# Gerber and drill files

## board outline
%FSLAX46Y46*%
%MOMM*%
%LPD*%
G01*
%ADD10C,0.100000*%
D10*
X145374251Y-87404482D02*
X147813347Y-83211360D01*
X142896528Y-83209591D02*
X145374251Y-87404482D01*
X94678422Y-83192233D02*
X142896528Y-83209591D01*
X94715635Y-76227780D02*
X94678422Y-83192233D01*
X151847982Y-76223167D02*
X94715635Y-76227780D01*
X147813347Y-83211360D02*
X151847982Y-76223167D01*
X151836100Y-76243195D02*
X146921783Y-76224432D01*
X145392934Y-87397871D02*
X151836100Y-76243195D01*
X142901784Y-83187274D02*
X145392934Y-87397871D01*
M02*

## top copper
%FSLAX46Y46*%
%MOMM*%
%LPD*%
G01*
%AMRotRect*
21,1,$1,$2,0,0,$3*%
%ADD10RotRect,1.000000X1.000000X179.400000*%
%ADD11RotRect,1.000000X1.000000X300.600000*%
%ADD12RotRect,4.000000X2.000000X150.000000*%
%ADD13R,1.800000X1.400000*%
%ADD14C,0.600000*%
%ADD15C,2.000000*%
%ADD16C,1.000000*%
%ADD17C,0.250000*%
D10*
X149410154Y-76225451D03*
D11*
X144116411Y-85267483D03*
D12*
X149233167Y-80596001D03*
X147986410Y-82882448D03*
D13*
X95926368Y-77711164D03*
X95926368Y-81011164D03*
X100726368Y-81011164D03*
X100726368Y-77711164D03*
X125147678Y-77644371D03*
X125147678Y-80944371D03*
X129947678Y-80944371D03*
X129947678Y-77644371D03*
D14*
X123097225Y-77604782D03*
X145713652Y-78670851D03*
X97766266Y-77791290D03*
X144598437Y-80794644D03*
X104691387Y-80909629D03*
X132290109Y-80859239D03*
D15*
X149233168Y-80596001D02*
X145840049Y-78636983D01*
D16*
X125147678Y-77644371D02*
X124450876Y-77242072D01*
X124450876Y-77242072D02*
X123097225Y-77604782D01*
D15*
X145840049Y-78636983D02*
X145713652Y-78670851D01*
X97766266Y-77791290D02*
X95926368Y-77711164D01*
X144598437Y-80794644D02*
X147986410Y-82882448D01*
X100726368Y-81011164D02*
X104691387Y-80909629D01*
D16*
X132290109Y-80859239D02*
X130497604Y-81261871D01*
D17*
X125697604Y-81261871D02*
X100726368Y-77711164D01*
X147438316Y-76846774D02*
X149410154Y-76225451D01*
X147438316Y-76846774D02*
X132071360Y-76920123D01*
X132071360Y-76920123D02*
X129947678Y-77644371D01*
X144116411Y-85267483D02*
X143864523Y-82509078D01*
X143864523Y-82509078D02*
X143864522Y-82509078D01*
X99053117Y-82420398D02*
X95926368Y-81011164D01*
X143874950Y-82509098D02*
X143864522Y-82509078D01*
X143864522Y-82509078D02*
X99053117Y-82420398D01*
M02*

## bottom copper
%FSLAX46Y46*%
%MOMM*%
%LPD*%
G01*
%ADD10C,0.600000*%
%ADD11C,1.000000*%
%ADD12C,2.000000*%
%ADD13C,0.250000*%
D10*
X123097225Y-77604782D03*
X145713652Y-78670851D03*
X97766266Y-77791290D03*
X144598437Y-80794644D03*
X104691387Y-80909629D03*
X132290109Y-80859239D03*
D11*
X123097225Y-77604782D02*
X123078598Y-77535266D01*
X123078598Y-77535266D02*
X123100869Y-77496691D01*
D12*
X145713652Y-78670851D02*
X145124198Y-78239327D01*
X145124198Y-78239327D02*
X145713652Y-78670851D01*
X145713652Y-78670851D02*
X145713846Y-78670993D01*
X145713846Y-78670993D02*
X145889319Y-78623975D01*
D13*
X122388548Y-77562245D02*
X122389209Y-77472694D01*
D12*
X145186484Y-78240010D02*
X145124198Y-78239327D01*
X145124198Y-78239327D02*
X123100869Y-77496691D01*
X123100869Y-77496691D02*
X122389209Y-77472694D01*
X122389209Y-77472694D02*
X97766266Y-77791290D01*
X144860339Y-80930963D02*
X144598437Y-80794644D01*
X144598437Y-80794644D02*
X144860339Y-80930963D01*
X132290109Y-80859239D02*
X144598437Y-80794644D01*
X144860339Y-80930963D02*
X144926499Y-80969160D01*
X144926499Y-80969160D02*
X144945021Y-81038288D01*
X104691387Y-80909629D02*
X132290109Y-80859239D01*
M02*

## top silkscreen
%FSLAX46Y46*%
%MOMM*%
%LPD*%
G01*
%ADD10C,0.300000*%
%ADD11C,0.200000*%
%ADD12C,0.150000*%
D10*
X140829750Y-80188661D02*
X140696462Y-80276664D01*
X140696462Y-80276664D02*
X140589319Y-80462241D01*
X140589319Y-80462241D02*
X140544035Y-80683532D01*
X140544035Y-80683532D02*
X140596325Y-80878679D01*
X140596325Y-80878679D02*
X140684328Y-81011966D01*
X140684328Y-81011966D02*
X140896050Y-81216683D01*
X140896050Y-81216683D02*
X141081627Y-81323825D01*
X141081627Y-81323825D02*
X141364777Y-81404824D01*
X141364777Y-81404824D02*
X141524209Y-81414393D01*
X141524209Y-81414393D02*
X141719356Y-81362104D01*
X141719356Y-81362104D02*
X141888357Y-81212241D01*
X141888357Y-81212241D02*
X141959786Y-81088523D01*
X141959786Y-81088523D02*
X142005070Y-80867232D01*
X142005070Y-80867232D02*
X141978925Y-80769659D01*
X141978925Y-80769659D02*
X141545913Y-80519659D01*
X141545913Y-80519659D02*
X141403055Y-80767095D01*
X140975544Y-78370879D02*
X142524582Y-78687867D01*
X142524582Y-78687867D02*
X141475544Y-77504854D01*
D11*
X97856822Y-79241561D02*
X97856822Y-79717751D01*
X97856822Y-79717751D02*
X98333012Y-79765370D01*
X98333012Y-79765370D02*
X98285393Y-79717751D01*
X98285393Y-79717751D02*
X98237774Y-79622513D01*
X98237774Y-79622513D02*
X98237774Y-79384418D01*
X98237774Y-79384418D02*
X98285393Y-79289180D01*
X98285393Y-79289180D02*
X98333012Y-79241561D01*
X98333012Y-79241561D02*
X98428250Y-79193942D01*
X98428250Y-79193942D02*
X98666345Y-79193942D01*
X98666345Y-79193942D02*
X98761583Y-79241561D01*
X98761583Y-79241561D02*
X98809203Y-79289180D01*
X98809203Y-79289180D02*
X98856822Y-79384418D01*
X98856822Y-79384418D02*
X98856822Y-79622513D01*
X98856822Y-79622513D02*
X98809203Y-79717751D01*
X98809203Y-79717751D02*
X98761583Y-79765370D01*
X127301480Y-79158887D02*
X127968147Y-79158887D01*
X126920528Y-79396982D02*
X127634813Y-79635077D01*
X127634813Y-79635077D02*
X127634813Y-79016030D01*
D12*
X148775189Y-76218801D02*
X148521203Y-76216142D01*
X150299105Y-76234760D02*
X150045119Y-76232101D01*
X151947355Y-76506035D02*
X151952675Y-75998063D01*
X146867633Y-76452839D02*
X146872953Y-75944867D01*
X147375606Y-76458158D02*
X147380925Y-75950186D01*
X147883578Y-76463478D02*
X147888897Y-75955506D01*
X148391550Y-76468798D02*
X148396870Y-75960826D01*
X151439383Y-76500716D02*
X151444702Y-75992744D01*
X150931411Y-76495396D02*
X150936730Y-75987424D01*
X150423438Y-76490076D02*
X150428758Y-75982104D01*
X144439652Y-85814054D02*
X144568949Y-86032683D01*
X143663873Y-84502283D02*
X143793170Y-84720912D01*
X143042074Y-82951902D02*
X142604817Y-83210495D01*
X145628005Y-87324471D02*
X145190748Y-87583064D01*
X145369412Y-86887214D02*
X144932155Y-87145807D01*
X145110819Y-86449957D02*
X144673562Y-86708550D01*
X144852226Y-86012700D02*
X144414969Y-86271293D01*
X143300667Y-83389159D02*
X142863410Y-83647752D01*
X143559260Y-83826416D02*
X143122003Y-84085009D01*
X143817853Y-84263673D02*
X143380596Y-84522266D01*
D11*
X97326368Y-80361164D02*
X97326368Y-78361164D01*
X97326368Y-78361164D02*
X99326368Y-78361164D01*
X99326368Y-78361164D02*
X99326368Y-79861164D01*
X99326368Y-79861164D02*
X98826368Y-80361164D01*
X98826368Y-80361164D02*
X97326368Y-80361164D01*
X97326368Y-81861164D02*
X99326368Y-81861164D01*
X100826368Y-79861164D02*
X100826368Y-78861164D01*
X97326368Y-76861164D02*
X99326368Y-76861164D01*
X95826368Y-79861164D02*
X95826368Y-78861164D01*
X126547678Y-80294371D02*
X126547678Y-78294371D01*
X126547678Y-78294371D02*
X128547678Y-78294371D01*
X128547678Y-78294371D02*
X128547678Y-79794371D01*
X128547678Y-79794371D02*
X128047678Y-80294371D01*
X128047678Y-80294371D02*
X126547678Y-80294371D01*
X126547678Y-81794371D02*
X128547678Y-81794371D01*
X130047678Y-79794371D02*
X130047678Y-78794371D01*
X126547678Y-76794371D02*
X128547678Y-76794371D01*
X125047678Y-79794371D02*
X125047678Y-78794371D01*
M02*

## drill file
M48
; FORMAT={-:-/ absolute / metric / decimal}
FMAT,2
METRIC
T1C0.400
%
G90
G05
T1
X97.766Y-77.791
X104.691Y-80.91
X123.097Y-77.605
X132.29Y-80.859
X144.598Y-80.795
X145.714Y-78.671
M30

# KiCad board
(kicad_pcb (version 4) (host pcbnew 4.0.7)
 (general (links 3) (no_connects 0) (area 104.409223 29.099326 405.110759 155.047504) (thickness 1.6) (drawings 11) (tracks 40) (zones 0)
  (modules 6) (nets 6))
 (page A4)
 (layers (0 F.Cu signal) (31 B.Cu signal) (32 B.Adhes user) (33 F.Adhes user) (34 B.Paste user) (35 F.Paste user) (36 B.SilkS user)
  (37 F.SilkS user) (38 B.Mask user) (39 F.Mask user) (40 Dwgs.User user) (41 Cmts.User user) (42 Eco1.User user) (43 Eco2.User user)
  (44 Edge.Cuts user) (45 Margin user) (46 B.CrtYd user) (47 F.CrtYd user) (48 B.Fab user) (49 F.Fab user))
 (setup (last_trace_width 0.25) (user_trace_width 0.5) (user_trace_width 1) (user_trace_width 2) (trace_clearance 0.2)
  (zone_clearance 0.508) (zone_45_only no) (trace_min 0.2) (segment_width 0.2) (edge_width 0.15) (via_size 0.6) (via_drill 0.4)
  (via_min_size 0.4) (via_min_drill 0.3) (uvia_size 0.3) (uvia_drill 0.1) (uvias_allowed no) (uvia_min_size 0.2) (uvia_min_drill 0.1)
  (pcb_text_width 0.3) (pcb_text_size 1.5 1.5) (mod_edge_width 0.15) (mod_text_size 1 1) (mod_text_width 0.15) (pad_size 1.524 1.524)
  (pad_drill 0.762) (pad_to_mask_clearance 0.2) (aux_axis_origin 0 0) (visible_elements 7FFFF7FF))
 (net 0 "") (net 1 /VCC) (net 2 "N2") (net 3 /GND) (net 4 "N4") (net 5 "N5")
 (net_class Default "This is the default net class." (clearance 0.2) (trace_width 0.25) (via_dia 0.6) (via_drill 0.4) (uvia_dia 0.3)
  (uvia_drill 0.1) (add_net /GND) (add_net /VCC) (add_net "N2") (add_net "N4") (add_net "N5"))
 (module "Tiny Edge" (layer F.Cu) (at 149.410153881754 76.2254514346474 179.4)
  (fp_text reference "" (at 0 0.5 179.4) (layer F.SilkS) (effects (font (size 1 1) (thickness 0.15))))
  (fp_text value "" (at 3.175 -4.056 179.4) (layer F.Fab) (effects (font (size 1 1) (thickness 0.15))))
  (fp_line (start 0.635 0) (end 0.889 0) (layer F.SilkS) (width 0.15))
  (fp_line (start -0.889 0) (end -0.635 0) (layer F.SilkS) (width 0.15))
  (fp_line (start -2.54 -0.254) (end -2.54 0.254) (layer F.SilkS) (width 0.15))
  (fp_line (start 2.54 -0.254) (end 2.54 0.254) (layer F.SilkS) (width 0.15))
  (fp_line (start 2.032 -0.254) (end 2.032 0.254) (layer F.SilkS) (width 0.15))
  (fp_line (start 1.524 -0.254) (end 1.524 0.254) (layer F.SilkS) (width 0.15))
  (fp_line (start 1.016 -0.254) (end 1.016 0.254) (layer F.SilkS) (width 0.15))
  (fp_line (start -2.032 -0.254) (end -2.032 0.254) (layer F.SilkS) (width 0.15))
  (fp_line (start -1.524 -0.254) (end -1.524 0.254) (layer F.SilkS) (width 0.15))
  (fp_line (start -1.016 -0.254) (end -1.016 0.254) (layer F.SilkS) (width 0.15))
  (pad 1 smd rect (at 0 0 179.4) (size 1 1) (layers F.Cu F.Paste F.Mask)))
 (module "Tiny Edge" (layer F.Cu) (at 144.116411268613 85.2674826027988 300.6)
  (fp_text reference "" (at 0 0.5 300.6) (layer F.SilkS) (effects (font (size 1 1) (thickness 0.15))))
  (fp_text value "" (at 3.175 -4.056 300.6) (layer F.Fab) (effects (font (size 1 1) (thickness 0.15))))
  (fp_line (start 0.635 0) (end 0.889 0) (layer F.SilkS) (width 0.15))
  (fp_line (start -0.889 0) (end -0.635 0) (layer F.SilkS) (width 0.15))
  (fp_line (start -2.54 -0.254) (end -2.54 0.254) (layer F.SilkS) (width 0.15))
  (fp_line (start 2.54 -0.254) (end 2.54 0.254) (layer F.SilkS) (width 0.15))
  (fp_line (start 2.032 -0.254) (end 2.032 0.254) (layer F.SilkS) (width 0.15))
  (fp_line (start 1.524 -0.254) (end 1.524 0.254) (layer F.SilkS) (width 0.15))
  (fp_line (start 1.016 -0.254) (end 1.016 0.254) (layer F.SilkS) (width 0.15))
  (fp_line (start -2.032 -0.254) (end -2.032 0.254) (layer F.SilkS) (width 0.15))
  (fp_line (start -1.524 -0.254) (end -1.524 0.254) (layer F.SilkS) (width 0.15))
  (fp_line (start -1.016 -0.254) (end -1.016 0.254) (layer F.SilkS) (width 0.15))
  (pad 1 smd rect (at 0 0 300.6) (size 1 1) (layers F.Cu F.Paste F.Mask)))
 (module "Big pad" (layer F.Cu) (at 149.186682275963 80.4225156099258 150)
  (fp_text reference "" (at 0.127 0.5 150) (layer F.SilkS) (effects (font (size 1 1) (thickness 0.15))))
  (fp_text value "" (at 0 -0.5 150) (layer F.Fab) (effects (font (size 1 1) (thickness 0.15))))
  (pad 1 smd rect (at -0.127 -0.127 150) (size 4 2) (layers F.Cu F.Paste F.Mask)))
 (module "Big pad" (layer F.Cu) (at 147.939924889103 82.7089627486785 150)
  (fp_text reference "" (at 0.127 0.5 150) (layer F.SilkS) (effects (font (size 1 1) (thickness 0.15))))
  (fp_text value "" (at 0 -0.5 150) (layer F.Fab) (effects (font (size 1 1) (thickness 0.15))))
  (pad 1 smd rect (at -0.127 -0.127 150) (size 4 2) (layers F.Cu F.Paste F.Mask)))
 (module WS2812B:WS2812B (layer F.Cu) (at 98.326367851464 79.3611642820861 90)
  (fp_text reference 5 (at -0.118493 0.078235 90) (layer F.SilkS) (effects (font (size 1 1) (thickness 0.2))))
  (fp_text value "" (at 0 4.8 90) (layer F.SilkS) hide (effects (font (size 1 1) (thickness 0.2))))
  (fp_line (start -1 -1) (end 1 -1) (layer F.SilkS) (width 0.2)) (fp_line (start 1 -1) (end 1 1) (layer F.SilkS) (width 0.2))
  (fp_line (start 1 1) (end -0.5 1) (layer F.SilkS) (width 0.2))
  (fp_line (start -0.5 1) (end -1 0.5) (layer F.SilkS) (width 0.2))
  (fp_line (start -1 0.5) (end -1 -1) (layer F.SilkS) (width 0.2))
  (fp_line (start -2.5 -1) (end -2.5 1) (layer F.SilkS) (width 0.2))
  (fp_line (start -0.5 2.5) (end 0.5 2.5) (layer F.SilkS) (width 0.2))
  (fp_line (start 2.5 -1) (end 2.5 1) (layer F.SilkS) (width 0.2))
  (fp_line (start -0.5 -2.5) (end 0.5 -2.5) (layer F.SilkS) (width 0.2))
  (pad 1 smd rect (at 1.65 -2.4 90) (size 1.4 1.8) (layers F.Cu F.Paste F.Mask) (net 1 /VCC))
  (pad 2 smd rect (at -1.65 -2.4 90) (size 1.4 1.8) (layers F.Cu F.Paste F.Mask) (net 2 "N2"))
  (pad 3 smd rect (at -1.65 2.4 90) (size 1.4 1.8) (layers F.Cu F.Paste F.Mask) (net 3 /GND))
  (pad 4 smd rect (at 1.65 2.4 90) (size 1.4 1.8) (layers F.Cu F.Paste F.Mask) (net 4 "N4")))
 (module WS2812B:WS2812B (layer F.Cu) (at 127.547677881308 79.2943706466741 90)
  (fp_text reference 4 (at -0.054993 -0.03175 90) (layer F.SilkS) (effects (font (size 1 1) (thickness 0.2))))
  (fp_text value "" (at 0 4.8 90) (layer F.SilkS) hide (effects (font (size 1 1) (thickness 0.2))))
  (fp_line (start -1 -1) (end 1 -1) (layer F.SilkS) (width 0.2)) (fp_line (start 1 -1) (end 1 1) (layer F.SilkS) (width 0.2))
  (fp_line (start 1 1) (end -0.5 1) (layer F.SilkS) (width 0.2))
  (fp_line (start -0.5 1) (end -1 0.5) (layer F.SilkS) (width 0.2))
  (fp_line (start -1 0.5) (end -1 -1) (layer F.SilkS) (width 0.2))
  (fp_line (start -2.5 -1) (end -2.5 1) (layer F.SilkS) (width 0.2))
  (fp_line (start -0.5 2.5) (end 0.5 2.5) (layer F.SilkS) (width 0.2))
  (fp_line (start 2.5 -1) (end 2.5 1) (layer F.SilkS) (width 0.2))
  (fp_line (start -0.5 -2.5) (end 0.5 -2.5) (layer F.SilkS) (width 0.2))
  (pad 1 smd rect (at 1.65 -2.4 90) (size 1.4 1.8) (layers F.Cu F.Paste F.Mask) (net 1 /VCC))
  (pad 2 smd rect (at -1.65 -2.4 90) (size 1.4 1.8) (layers F.Cu F.Paste F.Mask) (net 4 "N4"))
  (pad 3 smd rect (at -1.65 2.4 90) (size 1.4 1.8) (layers F.Cu F.Paste F.Mask) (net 3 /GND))
  (pad 4 smd rect (at 1.65 2.4 90) (size 1.4 1.8) (layers F.Cu F.Paste F.Mask) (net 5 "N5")))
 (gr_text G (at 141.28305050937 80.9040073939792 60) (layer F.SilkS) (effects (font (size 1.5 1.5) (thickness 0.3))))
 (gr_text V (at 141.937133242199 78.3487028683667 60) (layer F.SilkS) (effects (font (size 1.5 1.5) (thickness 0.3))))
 (gr_line (start 145.374251071433 87.404482156533) (end 147.813346899746 83.2113602573658) (layer Edge.Cuts) (width 0.1))
 (gr_line (start 142.896527855663 83.2095906533395) (end 145.374251071433 87.404482156533) (layer Edge.Cuts) (width 0.1))
 (gr_line (start 94.6784222433107 83.1922334186553) (end 142.896527855663 83.2095906533395) (layer Edge.Cuts) (width 0.1))
 (gr_line (start 94.7156346002544 76.2277797257594) (end 94.6784222433107 83.1922334186553) (layer Edge.Cuts) (width 0.1))
 (gr_line (start 151.847982399746 76.2231665813448) (end 94.7156346002544 76.2277797257594) (layer Edge.Cuts) (width 0.1))
 (gr_line (start 147.813346899746 83.2113602573658) (end 151.847982399746 76.2231665813448) (layer Edge.Cuts) (width 0.1))
 (gr_line (start 151.836100376734 76.2431948488973) (end 146.921783391845 76.2244315512234) (layer Edge.Cuts) (width 0.1))
 (gr_line (start 145.392933782481 87.3978707517741) (end 151.836100376734 76.2431948488973) (layer Edge.Cuts) (width 0.1))
 (gr_line (start 142.901784391845 83.1872740655994) (end 145.392933782481 87.3978707517741) (layer Edge.Cuts) (width 0.1))
 (segment (start 149.233167502244 80.5960008362064) (end 145.840048793302 78.6369828362064) (width 2) (layer F.Cu) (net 1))
 (segment (start 125.147677896411 77.6443705586809) (end 124.450876454602 77.2420720586809) (width 1) (layer F.Cu) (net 1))
 (segment (start 124.450876454602 77.2420720586809) (end 123.097224508925 77.6047820043578) (width 1) (layer F.Cu) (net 1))
 (via (at 123.097224508925 77.6047820043578) (size 0.6) (drill 0.4) (layers F.Cu B.Cu) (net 1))
 (segment (start 123.097224508925 77.6047820043578) (end 123.078597842152 77.5352663375846) (width 1) (layer B.Cu) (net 1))
 (segment (start 123.078597842152 77.5352663375846) (end 123.100869342152 77.4966909680239) (width 1) (layer B.Cu) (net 1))
 (via (at 145.713651828715 78.6708508007931) (size 0.6) (drill 0.4) (layers F.Cu B.Cu) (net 1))
 (segment (start 145.840048793302 78.6369828362064) (end 145.713651828715 78.6708508007931) (width 2) (layer F.Cu) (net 1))
 (segment (start 145.713651828715 78.6708508007931) (end 145.124198075369 78.2393266503006) (width 2) (layer B.Cu) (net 1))
 (segment (start 145.124198075369 78.2393266503006) (end 145.713651828715 78.6708508007931) (width 2) (layer B.Cu) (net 1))
 (segment (start 145.713651828715 78.6708508007931) (end 145.713845808786 78.6709928174536) (width 2) (layer B.Cu) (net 1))
 (segment (start 145.713845808786 78.6709928174536) (end 145.889318602029 78.6239750242105) (width 2) (layer B.Cu) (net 1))
 (segment (start 122.388548377522 77.5622450700594) (end 122.389208590573 77.472693547511) (width 0.25) (layer B.Cu) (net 1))
 (segment (start 145.186484032362 78.2400102081896) (end 145.124198075369 78.2393266503006) (width 2) (layer B.Cu) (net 1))
 (segment (start 145.124198075369 78.2393266503006) (end 123.100869342152 77.4966909680239) (width 2) (layer B.Cu) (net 1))
 (segment (start 123.100869342152 77.4966909680239) (end 122.389208590573 77.472693547511) (width 2) (layer B.Cu) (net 1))
 (segment (start 122.389208590573 77.472693547511) (end 97.7662655886577 77.7912898587008) (width 2) (layer B.Cu) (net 1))
 (via (at 97.7662655886577 77.7912898587008) (size 0.6) (drill 0.4) (layers F.Cu B.Cu) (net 1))
 (segment (start 97.7662655886577 77.7912898587008) (end 95.9263678665666 77.7111641940929) (width 2) (layer F.Cu) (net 1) (status 20))
 (segment (start 144.860338553246 80.9309627486785) (end 144.598436941815 80.7946436462603) (width 2) (layer B.Cu) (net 3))
 (via (at 144.598436941815 80.7946436462603) (size 0.6) (drill 0.4) (layers F.Cu B.Cu) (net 3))
 (segment (start 144.598436941815 80.7946436462603) (end 147.986410115384 82.8824479749592) (width 2) (layer F.Cu) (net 3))
 (segment (start 144.598436941815 80.7946436462603) (end 144.860338553246 80.9309627486785) (width 2) (layer B.Cu) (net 3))
 (segment (start 132.290109093112 80.8592388364291) (end 144.598436941815 80.7946436462603) (width 2) (layer B.Cu) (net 3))
 (segment (start 144.860338553246 80.9309627486785) (end 144.926498563968 80.9691602486785) (width 2) (layer B.Cu) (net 3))
 (segment (start 144.926498563968 80.9691602486785) (end 144.945021279526 81.038287964237) (width 2) (layer B.Cu) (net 3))
 (segment (start 100.726367836361 81.0111643700793) (end 104.691386552355 80.9096285010171) (width 2) (layer F.Cu) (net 3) (status 10))
 (segment (start 104.691386552355 80.9096285010171) (end 132.290109093112 80.8592388364291) (width 2) (layer B.Cu) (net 3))
 (via (at 104.691386552355 80.9096285010171) (size 0.6) (drill 0.4) (layers F.Cu B.Cu) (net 3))
 (segment (start 132.290109093112 80.8592388364291) (end 130.497603997609 81.2618707346673) (width 1) (layer F.Cu) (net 3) (status 20))
 (via (at 132.290109093112 80.8592388364291) (size 0.6) (drill 0.4) (layers F.Cu B.Cu) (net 3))
 (segment (start 125.697603944058 81.26187070375) (end 100.726367920117 77.7111642250103) (width 0.25) (layer F.Cu) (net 4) (status 10))
 (segment (start 147.438316392667 76.8467741500148) (end 149.410153881754 76.2254514346474) (width 0.25) (layer F.Cu) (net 5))
 (segment (start 147.438316392667 76.8467741500148) (end 132.071360246341 76.9201229531329) (width 0.25) (layer F.Cu) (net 5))
 (segment (start 132.071360246341 76.9201229531329) (end 129.947677949961 77.6443705895982) (width 0.25) (layer F.Cu) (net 5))
 (segment (start 144.116411268613 85.2674826027988) (end 143.864522786031 82.5090782524734) (width 0.25) (layer F.Cu) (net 2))
 (segment (start 143.864522786031 82.5090782524734) (end 143.864521920005 82.5090777524734) (width 0.25) (layer F.Cu) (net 2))
 (segment (start 99.0531166982346 82.4203983551374) (end 95.9263677828109 81.011164339162) (width 0.25) (layer F.Cu) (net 2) (status 20))
 (segment (start 143.874949655681 82.5090983844753) (end 143.864521920005 82.5090777524734) (width 0.25) (layer F.Cu) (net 2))
 (segment (start 143.864521920005 82.5090777524734) (end 99.0531166982346 82.4203983551374) (width 0.25) (layer F.Cu) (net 2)))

